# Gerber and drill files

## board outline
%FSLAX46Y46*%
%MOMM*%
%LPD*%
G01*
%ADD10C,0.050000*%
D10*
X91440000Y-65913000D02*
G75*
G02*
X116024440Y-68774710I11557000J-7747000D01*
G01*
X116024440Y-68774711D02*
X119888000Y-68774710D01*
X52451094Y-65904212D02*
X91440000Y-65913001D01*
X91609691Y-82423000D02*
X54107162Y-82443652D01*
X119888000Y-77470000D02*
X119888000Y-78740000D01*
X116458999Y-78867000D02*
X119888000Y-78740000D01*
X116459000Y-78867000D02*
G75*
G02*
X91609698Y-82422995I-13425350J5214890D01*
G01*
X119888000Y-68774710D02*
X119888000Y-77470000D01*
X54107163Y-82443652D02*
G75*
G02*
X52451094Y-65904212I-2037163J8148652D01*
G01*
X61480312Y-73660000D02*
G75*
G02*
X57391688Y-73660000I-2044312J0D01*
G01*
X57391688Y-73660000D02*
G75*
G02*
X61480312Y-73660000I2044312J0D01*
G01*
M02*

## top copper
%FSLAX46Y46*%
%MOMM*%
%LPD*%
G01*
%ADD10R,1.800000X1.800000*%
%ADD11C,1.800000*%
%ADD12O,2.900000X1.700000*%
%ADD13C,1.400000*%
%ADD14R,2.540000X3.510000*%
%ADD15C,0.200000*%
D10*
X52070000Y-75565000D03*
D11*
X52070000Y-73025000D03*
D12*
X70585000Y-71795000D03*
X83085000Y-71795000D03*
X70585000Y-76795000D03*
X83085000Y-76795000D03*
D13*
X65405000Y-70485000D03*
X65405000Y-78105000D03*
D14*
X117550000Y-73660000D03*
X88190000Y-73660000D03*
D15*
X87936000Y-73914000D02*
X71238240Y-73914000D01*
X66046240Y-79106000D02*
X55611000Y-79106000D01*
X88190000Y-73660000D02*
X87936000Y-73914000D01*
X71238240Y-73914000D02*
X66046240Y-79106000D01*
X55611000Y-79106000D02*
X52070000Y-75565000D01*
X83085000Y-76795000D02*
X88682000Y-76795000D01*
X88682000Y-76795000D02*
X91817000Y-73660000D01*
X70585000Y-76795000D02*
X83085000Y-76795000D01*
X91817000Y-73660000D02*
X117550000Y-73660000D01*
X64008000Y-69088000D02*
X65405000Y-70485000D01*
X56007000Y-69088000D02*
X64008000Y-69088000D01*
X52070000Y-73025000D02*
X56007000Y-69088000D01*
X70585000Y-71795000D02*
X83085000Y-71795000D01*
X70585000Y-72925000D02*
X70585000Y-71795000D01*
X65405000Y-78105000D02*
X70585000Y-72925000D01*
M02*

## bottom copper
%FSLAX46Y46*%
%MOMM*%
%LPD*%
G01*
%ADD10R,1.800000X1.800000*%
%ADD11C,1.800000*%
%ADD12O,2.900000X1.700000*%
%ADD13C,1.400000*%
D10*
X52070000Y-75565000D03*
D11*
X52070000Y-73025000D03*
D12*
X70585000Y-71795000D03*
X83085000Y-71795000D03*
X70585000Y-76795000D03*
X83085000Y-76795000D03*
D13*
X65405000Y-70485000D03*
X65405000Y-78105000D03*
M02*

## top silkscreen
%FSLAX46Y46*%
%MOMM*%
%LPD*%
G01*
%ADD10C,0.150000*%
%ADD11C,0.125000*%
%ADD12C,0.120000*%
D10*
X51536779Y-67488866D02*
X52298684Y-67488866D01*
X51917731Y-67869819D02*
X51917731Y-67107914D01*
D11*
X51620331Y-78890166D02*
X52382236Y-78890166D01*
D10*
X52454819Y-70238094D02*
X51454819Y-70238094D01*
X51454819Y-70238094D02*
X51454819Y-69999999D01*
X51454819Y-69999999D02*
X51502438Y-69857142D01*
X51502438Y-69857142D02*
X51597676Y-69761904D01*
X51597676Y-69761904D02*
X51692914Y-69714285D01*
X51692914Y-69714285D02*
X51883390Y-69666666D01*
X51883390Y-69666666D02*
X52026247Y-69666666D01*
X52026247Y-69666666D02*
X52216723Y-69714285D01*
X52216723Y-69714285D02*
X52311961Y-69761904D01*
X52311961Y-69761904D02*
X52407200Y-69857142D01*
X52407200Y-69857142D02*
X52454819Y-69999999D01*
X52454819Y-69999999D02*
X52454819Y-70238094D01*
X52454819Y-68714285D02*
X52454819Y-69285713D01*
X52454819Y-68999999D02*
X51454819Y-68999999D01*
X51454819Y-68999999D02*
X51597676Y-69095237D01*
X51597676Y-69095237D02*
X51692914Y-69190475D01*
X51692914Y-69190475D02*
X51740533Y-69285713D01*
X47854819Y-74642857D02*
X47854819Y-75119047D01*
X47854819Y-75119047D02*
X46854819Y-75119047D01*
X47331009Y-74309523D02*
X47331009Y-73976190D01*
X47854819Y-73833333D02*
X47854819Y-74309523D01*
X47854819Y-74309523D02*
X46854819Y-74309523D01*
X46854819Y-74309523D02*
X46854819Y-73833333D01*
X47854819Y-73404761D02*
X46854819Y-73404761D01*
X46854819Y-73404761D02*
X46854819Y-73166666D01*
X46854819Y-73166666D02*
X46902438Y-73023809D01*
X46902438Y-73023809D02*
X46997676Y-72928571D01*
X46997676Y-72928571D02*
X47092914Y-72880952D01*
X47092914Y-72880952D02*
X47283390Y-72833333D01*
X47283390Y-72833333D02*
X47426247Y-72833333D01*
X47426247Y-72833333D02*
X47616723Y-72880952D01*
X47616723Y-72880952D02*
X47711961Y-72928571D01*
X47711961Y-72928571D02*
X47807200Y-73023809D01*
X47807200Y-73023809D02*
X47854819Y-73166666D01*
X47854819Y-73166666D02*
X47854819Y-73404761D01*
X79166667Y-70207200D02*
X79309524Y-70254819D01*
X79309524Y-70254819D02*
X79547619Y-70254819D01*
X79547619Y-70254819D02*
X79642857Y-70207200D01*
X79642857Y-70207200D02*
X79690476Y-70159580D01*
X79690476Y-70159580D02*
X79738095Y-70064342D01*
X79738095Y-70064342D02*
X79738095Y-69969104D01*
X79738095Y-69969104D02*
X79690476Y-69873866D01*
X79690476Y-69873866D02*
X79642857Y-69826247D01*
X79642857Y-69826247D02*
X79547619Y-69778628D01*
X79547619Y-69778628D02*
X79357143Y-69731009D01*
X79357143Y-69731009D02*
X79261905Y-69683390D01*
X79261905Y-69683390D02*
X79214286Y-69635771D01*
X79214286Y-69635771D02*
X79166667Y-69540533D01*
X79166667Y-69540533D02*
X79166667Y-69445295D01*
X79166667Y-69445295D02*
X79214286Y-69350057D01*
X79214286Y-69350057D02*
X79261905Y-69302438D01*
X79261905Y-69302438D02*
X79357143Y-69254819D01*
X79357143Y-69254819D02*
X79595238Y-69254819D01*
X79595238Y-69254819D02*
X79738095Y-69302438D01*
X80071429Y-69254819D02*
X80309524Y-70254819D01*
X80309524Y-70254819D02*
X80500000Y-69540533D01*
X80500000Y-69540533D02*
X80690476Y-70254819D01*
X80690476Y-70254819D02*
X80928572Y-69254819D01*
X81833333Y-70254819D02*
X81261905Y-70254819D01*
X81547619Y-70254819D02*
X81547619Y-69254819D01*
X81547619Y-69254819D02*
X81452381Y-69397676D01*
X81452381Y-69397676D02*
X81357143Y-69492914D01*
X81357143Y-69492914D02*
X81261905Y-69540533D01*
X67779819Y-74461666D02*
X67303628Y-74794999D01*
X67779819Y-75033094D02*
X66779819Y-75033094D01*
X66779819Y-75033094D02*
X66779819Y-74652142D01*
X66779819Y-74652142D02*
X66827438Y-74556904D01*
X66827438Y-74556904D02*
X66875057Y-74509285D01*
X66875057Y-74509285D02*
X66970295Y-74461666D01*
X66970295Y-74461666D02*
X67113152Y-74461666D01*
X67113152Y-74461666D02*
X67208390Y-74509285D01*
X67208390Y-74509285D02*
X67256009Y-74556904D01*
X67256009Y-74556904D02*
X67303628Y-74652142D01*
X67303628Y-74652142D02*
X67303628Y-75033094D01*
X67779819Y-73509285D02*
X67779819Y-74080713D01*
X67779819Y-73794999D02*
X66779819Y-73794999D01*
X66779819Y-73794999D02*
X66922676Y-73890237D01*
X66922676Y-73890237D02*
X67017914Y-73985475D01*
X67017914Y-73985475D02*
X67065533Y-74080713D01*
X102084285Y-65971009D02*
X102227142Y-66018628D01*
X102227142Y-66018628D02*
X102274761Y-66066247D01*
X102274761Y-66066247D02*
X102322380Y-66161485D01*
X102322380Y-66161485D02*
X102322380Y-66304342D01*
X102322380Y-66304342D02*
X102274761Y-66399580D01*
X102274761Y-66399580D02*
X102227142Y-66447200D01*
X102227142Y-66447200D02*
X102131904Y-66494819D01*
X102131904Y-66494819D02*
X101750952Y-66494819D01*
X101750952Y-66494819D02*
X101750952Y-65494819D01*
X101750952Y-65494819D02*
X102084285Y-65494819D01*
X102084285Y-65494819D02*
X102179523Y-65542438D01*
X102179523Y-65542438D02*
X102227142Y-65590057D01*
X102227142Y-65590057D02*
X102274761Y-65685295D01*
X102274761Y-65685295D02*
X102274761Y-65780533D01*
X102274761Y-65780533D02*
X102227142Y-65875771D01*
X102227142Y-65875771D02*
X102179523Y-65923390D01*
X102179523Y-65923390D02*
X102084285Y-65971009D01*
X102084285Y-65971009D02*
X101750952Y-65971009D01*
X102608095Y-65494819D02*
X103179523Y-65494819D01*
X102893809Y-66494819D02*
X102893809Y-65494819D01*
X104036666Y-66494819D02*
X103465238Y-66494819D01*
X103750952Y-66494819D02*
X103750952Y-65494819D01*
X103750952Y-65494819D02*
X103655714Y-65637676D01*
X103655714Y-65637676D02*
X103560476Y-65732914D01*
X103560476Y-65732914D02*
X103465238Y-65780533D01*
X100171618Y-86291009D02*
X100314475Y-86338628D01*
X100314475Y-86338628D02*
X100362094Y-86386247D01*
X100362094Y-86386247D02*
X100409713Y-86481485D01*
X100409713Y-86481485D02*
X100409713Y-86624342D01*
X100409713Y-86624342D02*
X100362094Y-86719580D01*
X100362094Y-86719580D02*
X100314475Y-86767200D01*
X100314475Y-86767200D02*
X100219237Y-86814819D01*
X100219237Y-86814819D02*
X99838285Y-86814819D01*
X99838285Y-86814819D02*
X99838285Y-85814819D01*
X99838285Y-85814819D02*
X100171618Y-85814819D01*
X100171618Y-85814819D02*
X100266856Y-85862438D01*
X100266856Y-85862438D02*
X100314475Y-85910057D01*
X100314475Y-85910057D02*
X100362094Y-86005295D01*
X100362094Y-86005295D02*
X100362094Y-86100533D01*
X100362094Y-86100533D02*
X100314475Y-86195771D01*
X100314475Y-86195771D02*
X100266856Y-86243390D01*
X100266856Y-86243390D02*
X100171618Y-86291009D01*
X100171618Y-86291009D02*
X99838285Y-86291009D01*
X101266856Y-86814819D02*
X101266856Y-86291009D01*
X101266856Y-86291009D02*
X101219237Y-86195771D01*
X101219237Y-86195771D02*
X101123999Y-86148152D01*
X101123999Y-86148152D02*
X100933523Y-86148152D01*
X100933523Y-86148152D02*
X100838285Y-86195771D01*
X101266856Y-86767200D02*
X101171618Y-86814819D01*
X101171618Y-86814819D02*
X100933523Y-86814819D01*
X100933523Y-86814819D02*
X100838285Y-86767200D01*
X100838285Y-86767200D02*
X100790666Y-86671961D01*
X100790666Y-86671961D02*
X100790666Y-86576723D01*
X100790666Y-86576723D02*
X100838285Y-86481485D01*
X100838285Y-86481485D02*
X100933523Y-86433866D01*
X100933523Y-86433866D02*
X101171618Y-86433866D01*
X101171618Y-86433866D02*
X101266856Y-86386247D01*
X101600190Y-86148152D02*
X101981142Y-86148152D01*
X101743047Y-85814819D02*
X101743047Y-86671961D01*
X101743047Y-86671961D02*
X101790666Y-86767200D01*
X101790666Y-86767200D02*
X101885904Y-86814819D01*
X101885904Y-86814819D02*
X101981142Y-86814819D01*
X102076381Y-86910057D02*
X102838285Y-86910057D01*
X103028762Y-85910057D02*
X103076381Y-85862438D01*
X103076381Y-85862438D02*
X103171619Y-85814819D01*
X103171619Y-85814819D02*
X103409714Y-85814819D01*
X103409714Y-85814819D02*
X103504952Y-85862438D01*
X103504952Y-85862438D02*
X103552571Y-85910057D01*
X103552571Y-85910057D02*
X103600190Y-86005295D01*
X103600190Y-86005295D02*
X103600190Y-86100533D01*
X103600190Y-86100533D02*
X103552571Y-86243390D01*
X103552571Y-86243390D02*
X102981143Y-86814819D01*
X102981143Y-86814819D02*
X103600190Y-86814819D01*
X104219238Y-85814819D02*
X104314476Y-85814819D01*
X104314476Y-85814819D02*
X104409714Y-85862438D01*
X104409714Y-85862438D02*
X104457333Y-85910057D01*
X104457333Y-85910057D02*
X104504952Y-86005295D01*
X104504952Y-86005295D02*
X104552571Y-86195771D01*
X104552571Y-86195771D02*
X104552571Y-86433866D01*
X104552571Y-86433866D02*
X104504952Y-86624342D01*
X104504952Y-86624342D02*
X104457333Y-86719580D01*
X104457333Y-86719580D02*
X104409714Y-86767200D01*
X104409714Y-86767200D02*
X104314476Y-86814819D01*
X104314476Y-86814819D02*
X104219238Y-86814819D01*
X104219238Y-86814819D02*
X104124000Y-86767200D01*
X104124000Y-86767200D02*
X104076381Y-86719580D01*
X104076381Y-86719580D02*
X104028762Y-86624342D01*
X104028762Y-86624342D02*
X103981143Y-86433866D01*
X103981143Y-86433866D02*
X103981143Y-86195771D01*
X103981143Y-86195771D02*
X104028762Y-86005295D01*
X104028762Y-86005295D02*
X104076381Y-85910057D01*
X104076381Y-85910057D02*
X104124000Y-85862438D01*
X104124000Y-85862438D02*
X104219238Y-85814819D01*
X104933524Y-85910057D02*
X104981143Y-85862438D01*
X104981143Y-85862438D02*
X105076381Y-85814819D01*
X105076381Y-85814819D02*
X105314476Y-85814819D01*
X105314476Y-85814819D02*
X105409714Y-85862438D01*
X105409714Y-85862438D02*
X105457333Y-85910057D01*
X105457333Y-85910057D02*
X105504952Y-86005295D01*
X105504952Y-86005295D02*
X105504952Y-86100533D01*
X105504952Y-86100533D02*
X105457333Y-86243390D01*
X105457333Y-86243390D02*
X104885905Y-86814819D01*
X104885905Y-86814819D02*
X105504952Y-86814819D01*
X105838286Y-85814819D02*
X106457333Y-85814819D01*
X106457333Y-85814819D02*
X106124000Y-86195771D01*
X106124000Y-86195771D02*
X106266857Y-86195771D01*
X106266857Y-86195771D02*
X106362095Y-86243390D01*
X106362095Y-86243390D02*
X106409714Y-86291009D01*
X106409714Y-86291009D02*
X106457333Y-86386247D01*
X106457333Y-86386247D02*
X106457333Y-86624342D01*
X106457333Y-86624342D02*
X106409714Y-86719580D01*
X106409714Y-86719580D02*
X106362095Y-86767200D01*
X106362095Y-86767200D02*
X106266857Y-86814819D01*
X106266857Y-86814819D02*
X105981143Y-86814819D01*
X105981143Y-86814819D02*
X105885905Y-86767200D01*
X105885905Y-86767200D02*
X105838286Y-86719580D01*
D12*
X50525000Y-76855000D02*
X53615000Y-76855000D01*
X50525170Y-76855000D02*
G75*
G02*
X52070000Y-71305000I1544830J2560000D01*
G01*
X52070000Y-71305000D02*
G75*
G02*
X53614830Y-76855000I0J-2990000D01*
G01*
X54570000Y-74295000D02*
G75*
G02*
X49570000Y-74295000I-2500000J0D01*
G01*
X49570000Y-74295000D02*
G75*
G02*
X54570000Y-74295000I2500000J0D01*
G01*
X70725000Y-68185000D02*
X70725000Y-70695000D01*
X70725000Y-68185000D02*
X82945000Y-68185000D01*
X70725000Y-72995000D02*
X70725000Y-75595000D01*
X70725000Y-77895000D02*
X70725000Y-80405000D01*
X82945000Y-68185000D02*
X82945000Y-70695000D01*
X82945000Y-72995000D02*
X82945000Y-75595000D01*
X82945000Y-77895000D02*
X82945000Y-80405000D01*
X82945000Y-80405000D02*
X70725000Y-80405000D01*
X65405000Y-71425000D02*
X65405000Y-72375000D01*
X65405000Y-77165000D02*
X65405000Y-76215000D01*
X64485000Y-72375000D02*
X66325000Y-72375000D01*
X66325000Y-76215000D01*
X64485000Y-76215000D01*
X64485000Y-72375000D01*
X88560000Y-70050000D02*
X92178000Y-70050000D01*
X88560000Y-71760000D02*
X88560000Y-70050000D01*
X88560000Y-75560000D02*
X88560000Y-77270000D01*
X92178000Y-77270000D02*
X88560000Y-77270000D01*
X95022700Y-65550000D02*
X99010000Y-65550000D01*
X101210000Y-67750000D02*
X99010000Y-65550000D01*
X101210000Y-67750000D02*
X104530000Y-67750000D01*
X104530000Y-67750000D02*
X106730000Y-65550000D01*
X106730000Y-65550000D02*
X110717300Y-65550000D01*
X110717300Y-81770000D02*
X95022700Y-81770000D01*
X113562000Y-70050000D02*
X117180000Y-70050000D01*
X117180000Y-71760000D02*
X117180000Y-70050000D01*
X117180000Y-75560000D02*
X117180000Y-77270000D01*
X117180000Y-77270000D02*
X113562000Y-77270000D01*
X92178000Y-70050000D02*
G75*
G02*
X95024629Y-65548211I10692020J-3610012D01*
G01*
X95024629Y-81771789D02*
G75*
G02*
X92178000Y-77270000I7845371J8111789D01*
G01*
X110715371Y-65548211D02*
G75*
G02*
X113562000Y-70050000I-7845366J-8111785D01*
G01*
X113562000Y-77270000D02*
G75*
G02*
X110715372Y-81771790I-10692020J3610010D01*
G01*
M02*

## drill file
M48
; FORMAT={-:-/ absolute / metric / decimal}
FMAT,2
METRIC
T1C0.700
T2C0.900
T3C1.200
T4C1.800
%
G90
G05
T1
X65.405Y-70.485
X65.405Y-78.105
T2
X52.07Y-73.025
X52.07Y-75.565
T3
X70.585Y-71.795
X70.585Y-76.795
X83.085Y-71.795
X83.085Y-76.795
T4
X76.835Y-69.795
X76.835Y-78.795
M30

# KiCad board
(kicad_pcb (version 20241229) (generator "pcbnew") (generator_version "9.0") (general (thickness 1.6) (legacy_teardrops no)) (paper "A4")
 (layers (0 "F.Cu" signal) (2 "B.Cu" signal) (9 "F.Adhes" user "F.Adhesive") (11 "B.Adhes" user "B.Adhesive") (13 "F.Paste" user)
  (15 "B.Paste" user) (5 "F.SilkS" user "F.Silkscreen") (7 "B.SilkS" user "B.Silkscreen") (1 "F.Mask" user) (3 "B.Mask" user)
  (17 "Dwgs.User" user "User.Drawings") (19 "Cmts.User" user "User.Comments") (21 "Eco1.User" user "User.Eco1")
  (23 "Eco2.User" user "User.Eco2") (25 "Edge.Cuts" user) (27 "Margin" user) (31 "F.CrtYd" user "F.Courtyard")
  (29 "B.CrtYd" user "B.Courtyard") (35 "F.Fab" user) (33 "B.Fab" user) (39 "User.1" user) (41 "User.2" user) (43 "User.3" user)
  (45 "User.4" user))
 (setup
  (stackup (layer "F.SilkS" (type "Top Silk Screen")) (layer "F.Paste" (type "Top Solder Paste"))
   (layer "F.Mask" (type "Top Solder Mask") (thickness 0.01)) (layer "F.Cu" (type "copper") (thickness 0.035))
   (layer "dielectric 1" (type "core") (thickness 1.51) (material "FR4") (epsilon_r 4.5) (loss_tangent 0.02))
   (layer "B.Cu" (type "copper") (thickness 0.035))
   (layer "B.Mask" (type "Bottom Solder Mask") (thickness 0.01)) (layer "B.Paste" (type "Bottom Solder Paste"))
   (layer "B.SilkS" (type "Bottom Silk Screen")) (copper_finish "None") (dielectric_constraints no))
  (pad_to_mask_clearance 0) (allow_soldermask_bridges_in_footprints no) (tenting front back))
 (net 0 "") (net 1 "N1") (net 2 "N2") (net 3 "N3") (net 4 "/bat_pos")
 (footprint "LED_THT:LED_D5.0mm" (layer "F.Cu") (at 52.07 75.565 90)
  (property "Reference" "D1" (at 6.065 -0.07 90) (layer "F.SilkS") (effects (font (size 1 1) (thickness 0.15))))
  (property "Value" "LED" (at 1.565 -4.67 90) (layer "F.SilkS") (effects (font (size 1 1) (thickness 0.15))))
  (fp_line (start -1.29 -1.545) (end -1.29 1.545) (stroke (width 0.12) (type solid)) (layer "F.SilkS"))
  (fp_arc (start -1.29 -1.54483) (mid 2.071779 -2.880495) (end 4.26 0) (stroke (width 0.12) (type solid)) (layer "F.SilkS"))
  (fp_arc (start 4.26 0) (mid 2.071779 2.880495) (end -1.29 1.54483) (stroke (width 0.12) (type solid)) (layer "F.SilkS"))
  (fp_circle (center 1.27 0) (end 3.77 0) (stroke (width 0.12) (type solid)) (fill no) (layer "F.SilkS"))
  (pad "1" thru_hole rect (at 0 0 90) (size 1.8 1.8) (drill 0.9) (layers "*.Cu" "*.Mask") (remove_unused_layers no) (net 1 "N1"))
  (pad "2" thru_hole circle (at 2.54 0 90) (size 1.8 1.8) (drill 0.9) (layers "*.Cu" "*.Mask") (remove_unused_layers no) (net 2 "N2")))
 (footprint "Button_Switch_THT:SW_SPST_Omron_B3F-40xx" (layer "F.Cu") (at 70.585 71.795)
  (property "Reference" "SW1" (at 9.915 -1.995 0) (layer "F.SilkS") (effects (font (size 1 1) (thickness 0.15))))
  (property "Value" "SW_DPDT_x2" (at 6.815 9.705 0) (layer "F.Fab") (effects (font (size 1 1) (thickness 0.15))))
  (fp_line (start 0.14 -3.61) (end 0.14 -1.1) (stroke (width 0.12) (type default)) (layer "F.SilkS"))
  (fp_line (start 0.14 -3.61) (end 12.36 -3.61) (stroke (width 0.12) (type default)) (layer "F.SilkS"))
  (fp_line (start 0.14 1.2) (end 0.14 3.8) (stroke (width 0.12) (type default)) (layer "F.SilkS"))
  (fp_line (start 0.14 6.1) (end 0.14 8.61) (stroke (width 0.12) (type default)) (layer "F.SilkS"))
  (fp_line (start 12.36 -3.61) (end 12.36 -1.1) (stroke (width 0.12) (type default)) (layer "F.SilkS"))
  (fp_line (start 12.36 1.2) (end 12.36 3.8) (stroke (width 0.12) (type default)) (layer "F.SilkS"))
  (fp_line (start 12.36 6.1) (end 12.36 8.61) (stroke (width 0.12) (type default)) (layer "F.SilkS"))
  (fp_line (start 12.36 8.61) (end 0.14 8.61) (stroke (width 0.12) (type default)) (layer "F.SilkS"))
  (pad "" np_thru_hole circle (at 6.25 -2) (size 1.8 1.8) (drill 1.8) (layers "*.Cu" "*.Mask"))
  (pad "" np_thru_hole circle (at 6.25 7) (size 1.8 1.8) (drill 1.8) (layers "*.Cu" "*.Mask"))
  (pad "1" thru_hole oval (at 0 0) (size 2.9 1.7) (drill 1.2) (layers "*.Cu" "*.Mask") (remove_unused_layers no) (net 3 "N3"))
  (pad "1" thru_hole oval (at 12.5 0) (size 2.9 1.7) (drill 1.2) (layers "*.Cu" "*.Mask") (remove_unused_layers no) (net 3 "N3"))
  (pad "2" thru_hole oval (at 0 5) (size 2.9 1.7) (drill 1.2) (layers "*.Cu" "*.Mask") (remove_unused_layers no) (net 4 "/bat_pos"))
  (pad "2" thru_hole oval (at 12.5 5) (size 2.9 1.7) (drill 1.2) (layers "*.Cu" "*.Mask") (remove_unused_layers no) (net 4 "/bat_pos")))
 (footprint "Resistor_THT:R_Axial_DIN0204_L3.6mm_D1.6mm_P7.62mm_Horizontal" (layer "F.Cu") (at 65.405 70.485 -90)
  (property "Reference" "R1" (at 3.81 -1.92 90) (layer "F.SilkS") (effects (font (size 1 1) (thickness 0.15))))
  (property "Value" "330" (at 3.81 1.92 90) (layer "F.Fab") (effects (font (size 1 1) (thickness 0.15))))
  (fp_line (start 0.94 0) (end 1.89 0) (stroke (width 0.12) (type solid)) (layer "F.SilkS"))
  (fp_line (start 6.68 0) (end 5.73 0) (stroke (width 0.12) (type solid)) (layer "F.SilkS"))
  (fp_rect (start 1.89 -0.92) (end 5.73 0.92) (stroke (width 0.12) (type solid)) (fill no) (layer "F.SilkS"))
  (pad "1" thru_hole circle (at 0 0 270) (size 1.4 1.4) (drill 0.7) (layers "*.Cu" "*.Mask") (remove_unused_layers no) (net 2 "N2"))
  (pad "2" thru_hole circle (at 7.62 0 270) (size 1.4 1.4) (drill 0.7) (layers "*.Cu" "*.Mask") (remove_unused_layers no) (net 3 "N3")))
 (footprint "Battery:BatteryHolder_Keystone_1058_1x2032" (layer "F.Cu") (at 102.87 73.66 180)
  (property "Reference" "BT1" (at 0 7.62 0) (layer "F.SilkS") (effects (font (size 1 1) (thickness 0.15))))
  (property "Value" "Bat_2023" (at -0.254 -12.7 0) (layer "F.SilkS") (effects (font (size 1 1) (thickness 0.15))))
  (fp_line (start 14.31 3.61) (end 10.692 3.61) (stroke (width 0.12) (type solid)) (layer "F.SilkS"))
  (fp_line (start 14.31 1.9) (end 14.31 3.61) (stroke (width 0.12) (type solid)) (layer "F.SilkS"))
  (fp_line (start 14.31 -1.9) (end 14.31 -3.61) (stroke (width 0.12) (type solid)) (layer "F.SilkS"))
  (fp_line (start 10.692 -3.61) (end 14.31 -3.61) (stroke (width 0.12) (type solid)) (layer "F.SilkS"))
  (fp_line (start 7.8473 8.11) (end 3.86 8.11) (stroke (width 0.12) (type solid)) (layer "F.SilkS"))
  (fp_line (start 1.66 5.91) (end 3.86 8.11) (stroke (width 0.12) (type solid)) (layer "F.SilkS"))
  (fp_line (start 1.66 5.91) (end -1.66 5.91) (stroke (width 0.12) (type solid)) (layer "F.SilkS"))
  (fp_line (start -1.66 5.91) (end -3.86 8.11) (stroke (width 0.12) (type solid)) (layer "F.SilkS"))
  (fp_line (start -3.86 8.11) (end -7.8473 8.11) (stroke (width 0.12) (type solid)) (layer "F.SilkS"))
  (fp_line (start -7.8473 -8.11) (end 7.8473 -8.11) (stroke (width 0.12) (type solid)) (layer "F.SilkS"))
  (fp_line (start -10.692 3.61) (end -14.31 3.61) (stroke (width 0.12) (type solid)) (layer "F.SilkS"))
  (fp_line (start -14.31 1.9) (end -14.31 3.61) (stroke (width 0.12) (type solid)) (layer "F.SilkS"))
  (fp_line (start -14.31 -1.9) (end -14.31 -3.61) (stroke (width 0.12) (type solid)) (layer "F.SilkS"))
  (fp_line (start -14.31 -3.61) (end -10.692 -3.61) (stroke (width 0.12) (type solid)) (layer "F.SilkS"))
  (fp_arc (start 10.692 3.61) (mid 9.538084 6.031244) (end 7.845371 8.111789) (stroke (width 0.12) (type solid)) (layer "F.SilkS"))
  (fp_arc (start 7.845371 -8.111789) (mid 9.538085 -6.031244) (end 10.692 -3.61) (stroke (width 0.12) (type solid)) (layer "F.SilkS"))
  (fp_arc (start -7.845371 8.111789) (mid -9.538085 6.031244) (end -10.692 3.61) (stroke (width 0.12) (type solid)) (layer "F.SilkS"))
  (fp_arc (start -10.692 -3.61) (mid -9.538084 -6.031244) (end -7.845371 -8.111789) (stroke (width 0.12) (type solid)) (layer "F.SilkS"))
  (pad "1" smd rect (at -14.68 0 180) (size 2.54 3.51) (layers "F.Cu" "F.Mask" "F.Paste") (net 4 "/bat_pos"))
  (pad "2" smd rect (at 14.68 0 180) (size 2.54 3.51) (layers "F.Cu" "F.Mask" "F.Paste") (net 1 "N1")))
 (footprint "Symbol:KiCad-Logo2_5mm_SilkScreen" (layer "B.Cu") (at 102.87 73.152 180)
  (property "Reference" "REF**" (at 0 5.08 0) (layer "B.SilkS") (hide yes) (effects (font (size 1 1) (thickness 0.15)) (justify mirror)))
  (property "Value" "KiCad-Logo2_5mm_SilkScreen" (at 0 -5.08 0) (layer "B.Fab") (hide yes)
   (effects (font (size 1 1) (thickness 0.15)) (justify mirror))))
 (gr_arc (start 91.44 65.913) (mid 104.605693 59.840001) (end 116.02444 68.77471) (stroke (width 0.05) (type default)) (locked yes)
  (layer "Edge.Cuts"))
 (gr_line (start 116.02444 68.774711) (end 119.888 68.77471) (stroke (width 0.05) (type default)) (locked yes) (layer "Edge.Cuts"))
 (gr_line (start 52.451094 65.904212) (end 91.44 65.913001) (stroke (width 0.05) (type default)) (locked yes) (layer "Edge.Cuts"))
 (gr_line (start 91.609691 82.423) (end 54.107162 82.443652) (stroke (width 0.05) (type default)) (locked yes) (layer "Edge.Cuts"))
 (gr_line (start 119.888 77.47) (end 119.888 78.74) (stroke (width 0.05) (type default)) (locked yes) (layer "Edge.Cuts"))
 (gr_line (start 116.458999 78.867) (end 119.888 78.74) (stroke (width 0.05) (type default)) (locked yes) (layer "Edge.Cuts"))
 (gr_arc (start 116.459 78.867) (mid 105.073913 87.90948) (end 91.609691 82.423) (stroke (width 0.05) (type default)) (locked yes)
  (layer "Edge.Cuts"))
 (gr_line (start 119.888 68.77471) (end 119.888 77.47) (stroke (width 0.05) (type default)) (locked yes) (layer "Edge.Cuts"))
 (gr_arc (start 54.107163 82.443652) (mid 43.712353 75.131838) (end 52.451094 65.904212) (stroke (width 0.05) (type default)) (locked yes)
  (layer "Edge.Cuts"))
 (gr_circle (center 59.436 73.66) (end 57.658 72.651077) (stroke (width 0.05) (type default)) (fill no) (locked yes) (layer "Edge.Cuts"))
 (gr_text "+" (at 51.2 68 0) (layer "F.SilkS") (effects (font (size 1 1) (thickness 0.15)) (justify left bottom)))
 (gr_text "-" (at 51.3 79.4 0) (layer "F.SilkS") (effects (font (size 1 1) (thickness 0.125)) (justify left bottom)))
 (segment (start 87.936 73.914) (end 71.23824 73.914) (width 0.2) (layer "F.Cu") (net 1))
 (segment (start 66.04624 79.106) (end 55.611 79.106) (width 0.2) (layer "F.Cu") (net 1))
 (segment (start 88.19 73.66) (end 87.936 73.914) (width 0.2) (layer "F.Cu") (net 1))
 (segment (start 71.23824 73.914) (end 66.04624 79.106) (width 0.2) (layer "F.Cu") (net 1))
 (segment (start 55.611 79.106) (end 52.07 75.565) (width 0.2) (layer "F.Cu") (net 1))
 (segment (start 83.085 76.795) (end 88.682 76.795) (width 0.2) (layer "F.Cu") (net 4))
 (segment (start 88.682 76.795) (end 91.817 73.66) (width 0.2) (layer "F.Cu") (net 4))
 (segment (start 70.585 76.795) (end 83.085 76.795) (width 0.2) (layer "F.Cu") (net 4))
 (segment (start 91.817 73.66) (end 117.55 73.66) (width 0.2) (layer "F.Cu") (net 4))
 (segment (start 64.008 69.088) (end 65.405 70.485) (width 0.2) (layer "F.Cu") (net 2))
 (segment (start 56.007 69.088) (end 64.008 69.088) (width 0.2) (layer "F.Cu") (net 2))
 (segment (start 52.07 73.025) (end 56.007 69.088) (width 0.2) (layer "F.Cu") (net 2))
 (segment (start 70.585 71.795) (end 83.085 71.795) (width 0.2) (layer "F.Cu") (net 3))
 (segment (start 70.585 72.925) (end 70.585 71.795) (width 0.2) (layer "F.Cu") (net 3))
 (segment (start 65.405 78.105) (end 70.585 72.925) (width 0.2) (layer "F.Cu") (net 3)))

